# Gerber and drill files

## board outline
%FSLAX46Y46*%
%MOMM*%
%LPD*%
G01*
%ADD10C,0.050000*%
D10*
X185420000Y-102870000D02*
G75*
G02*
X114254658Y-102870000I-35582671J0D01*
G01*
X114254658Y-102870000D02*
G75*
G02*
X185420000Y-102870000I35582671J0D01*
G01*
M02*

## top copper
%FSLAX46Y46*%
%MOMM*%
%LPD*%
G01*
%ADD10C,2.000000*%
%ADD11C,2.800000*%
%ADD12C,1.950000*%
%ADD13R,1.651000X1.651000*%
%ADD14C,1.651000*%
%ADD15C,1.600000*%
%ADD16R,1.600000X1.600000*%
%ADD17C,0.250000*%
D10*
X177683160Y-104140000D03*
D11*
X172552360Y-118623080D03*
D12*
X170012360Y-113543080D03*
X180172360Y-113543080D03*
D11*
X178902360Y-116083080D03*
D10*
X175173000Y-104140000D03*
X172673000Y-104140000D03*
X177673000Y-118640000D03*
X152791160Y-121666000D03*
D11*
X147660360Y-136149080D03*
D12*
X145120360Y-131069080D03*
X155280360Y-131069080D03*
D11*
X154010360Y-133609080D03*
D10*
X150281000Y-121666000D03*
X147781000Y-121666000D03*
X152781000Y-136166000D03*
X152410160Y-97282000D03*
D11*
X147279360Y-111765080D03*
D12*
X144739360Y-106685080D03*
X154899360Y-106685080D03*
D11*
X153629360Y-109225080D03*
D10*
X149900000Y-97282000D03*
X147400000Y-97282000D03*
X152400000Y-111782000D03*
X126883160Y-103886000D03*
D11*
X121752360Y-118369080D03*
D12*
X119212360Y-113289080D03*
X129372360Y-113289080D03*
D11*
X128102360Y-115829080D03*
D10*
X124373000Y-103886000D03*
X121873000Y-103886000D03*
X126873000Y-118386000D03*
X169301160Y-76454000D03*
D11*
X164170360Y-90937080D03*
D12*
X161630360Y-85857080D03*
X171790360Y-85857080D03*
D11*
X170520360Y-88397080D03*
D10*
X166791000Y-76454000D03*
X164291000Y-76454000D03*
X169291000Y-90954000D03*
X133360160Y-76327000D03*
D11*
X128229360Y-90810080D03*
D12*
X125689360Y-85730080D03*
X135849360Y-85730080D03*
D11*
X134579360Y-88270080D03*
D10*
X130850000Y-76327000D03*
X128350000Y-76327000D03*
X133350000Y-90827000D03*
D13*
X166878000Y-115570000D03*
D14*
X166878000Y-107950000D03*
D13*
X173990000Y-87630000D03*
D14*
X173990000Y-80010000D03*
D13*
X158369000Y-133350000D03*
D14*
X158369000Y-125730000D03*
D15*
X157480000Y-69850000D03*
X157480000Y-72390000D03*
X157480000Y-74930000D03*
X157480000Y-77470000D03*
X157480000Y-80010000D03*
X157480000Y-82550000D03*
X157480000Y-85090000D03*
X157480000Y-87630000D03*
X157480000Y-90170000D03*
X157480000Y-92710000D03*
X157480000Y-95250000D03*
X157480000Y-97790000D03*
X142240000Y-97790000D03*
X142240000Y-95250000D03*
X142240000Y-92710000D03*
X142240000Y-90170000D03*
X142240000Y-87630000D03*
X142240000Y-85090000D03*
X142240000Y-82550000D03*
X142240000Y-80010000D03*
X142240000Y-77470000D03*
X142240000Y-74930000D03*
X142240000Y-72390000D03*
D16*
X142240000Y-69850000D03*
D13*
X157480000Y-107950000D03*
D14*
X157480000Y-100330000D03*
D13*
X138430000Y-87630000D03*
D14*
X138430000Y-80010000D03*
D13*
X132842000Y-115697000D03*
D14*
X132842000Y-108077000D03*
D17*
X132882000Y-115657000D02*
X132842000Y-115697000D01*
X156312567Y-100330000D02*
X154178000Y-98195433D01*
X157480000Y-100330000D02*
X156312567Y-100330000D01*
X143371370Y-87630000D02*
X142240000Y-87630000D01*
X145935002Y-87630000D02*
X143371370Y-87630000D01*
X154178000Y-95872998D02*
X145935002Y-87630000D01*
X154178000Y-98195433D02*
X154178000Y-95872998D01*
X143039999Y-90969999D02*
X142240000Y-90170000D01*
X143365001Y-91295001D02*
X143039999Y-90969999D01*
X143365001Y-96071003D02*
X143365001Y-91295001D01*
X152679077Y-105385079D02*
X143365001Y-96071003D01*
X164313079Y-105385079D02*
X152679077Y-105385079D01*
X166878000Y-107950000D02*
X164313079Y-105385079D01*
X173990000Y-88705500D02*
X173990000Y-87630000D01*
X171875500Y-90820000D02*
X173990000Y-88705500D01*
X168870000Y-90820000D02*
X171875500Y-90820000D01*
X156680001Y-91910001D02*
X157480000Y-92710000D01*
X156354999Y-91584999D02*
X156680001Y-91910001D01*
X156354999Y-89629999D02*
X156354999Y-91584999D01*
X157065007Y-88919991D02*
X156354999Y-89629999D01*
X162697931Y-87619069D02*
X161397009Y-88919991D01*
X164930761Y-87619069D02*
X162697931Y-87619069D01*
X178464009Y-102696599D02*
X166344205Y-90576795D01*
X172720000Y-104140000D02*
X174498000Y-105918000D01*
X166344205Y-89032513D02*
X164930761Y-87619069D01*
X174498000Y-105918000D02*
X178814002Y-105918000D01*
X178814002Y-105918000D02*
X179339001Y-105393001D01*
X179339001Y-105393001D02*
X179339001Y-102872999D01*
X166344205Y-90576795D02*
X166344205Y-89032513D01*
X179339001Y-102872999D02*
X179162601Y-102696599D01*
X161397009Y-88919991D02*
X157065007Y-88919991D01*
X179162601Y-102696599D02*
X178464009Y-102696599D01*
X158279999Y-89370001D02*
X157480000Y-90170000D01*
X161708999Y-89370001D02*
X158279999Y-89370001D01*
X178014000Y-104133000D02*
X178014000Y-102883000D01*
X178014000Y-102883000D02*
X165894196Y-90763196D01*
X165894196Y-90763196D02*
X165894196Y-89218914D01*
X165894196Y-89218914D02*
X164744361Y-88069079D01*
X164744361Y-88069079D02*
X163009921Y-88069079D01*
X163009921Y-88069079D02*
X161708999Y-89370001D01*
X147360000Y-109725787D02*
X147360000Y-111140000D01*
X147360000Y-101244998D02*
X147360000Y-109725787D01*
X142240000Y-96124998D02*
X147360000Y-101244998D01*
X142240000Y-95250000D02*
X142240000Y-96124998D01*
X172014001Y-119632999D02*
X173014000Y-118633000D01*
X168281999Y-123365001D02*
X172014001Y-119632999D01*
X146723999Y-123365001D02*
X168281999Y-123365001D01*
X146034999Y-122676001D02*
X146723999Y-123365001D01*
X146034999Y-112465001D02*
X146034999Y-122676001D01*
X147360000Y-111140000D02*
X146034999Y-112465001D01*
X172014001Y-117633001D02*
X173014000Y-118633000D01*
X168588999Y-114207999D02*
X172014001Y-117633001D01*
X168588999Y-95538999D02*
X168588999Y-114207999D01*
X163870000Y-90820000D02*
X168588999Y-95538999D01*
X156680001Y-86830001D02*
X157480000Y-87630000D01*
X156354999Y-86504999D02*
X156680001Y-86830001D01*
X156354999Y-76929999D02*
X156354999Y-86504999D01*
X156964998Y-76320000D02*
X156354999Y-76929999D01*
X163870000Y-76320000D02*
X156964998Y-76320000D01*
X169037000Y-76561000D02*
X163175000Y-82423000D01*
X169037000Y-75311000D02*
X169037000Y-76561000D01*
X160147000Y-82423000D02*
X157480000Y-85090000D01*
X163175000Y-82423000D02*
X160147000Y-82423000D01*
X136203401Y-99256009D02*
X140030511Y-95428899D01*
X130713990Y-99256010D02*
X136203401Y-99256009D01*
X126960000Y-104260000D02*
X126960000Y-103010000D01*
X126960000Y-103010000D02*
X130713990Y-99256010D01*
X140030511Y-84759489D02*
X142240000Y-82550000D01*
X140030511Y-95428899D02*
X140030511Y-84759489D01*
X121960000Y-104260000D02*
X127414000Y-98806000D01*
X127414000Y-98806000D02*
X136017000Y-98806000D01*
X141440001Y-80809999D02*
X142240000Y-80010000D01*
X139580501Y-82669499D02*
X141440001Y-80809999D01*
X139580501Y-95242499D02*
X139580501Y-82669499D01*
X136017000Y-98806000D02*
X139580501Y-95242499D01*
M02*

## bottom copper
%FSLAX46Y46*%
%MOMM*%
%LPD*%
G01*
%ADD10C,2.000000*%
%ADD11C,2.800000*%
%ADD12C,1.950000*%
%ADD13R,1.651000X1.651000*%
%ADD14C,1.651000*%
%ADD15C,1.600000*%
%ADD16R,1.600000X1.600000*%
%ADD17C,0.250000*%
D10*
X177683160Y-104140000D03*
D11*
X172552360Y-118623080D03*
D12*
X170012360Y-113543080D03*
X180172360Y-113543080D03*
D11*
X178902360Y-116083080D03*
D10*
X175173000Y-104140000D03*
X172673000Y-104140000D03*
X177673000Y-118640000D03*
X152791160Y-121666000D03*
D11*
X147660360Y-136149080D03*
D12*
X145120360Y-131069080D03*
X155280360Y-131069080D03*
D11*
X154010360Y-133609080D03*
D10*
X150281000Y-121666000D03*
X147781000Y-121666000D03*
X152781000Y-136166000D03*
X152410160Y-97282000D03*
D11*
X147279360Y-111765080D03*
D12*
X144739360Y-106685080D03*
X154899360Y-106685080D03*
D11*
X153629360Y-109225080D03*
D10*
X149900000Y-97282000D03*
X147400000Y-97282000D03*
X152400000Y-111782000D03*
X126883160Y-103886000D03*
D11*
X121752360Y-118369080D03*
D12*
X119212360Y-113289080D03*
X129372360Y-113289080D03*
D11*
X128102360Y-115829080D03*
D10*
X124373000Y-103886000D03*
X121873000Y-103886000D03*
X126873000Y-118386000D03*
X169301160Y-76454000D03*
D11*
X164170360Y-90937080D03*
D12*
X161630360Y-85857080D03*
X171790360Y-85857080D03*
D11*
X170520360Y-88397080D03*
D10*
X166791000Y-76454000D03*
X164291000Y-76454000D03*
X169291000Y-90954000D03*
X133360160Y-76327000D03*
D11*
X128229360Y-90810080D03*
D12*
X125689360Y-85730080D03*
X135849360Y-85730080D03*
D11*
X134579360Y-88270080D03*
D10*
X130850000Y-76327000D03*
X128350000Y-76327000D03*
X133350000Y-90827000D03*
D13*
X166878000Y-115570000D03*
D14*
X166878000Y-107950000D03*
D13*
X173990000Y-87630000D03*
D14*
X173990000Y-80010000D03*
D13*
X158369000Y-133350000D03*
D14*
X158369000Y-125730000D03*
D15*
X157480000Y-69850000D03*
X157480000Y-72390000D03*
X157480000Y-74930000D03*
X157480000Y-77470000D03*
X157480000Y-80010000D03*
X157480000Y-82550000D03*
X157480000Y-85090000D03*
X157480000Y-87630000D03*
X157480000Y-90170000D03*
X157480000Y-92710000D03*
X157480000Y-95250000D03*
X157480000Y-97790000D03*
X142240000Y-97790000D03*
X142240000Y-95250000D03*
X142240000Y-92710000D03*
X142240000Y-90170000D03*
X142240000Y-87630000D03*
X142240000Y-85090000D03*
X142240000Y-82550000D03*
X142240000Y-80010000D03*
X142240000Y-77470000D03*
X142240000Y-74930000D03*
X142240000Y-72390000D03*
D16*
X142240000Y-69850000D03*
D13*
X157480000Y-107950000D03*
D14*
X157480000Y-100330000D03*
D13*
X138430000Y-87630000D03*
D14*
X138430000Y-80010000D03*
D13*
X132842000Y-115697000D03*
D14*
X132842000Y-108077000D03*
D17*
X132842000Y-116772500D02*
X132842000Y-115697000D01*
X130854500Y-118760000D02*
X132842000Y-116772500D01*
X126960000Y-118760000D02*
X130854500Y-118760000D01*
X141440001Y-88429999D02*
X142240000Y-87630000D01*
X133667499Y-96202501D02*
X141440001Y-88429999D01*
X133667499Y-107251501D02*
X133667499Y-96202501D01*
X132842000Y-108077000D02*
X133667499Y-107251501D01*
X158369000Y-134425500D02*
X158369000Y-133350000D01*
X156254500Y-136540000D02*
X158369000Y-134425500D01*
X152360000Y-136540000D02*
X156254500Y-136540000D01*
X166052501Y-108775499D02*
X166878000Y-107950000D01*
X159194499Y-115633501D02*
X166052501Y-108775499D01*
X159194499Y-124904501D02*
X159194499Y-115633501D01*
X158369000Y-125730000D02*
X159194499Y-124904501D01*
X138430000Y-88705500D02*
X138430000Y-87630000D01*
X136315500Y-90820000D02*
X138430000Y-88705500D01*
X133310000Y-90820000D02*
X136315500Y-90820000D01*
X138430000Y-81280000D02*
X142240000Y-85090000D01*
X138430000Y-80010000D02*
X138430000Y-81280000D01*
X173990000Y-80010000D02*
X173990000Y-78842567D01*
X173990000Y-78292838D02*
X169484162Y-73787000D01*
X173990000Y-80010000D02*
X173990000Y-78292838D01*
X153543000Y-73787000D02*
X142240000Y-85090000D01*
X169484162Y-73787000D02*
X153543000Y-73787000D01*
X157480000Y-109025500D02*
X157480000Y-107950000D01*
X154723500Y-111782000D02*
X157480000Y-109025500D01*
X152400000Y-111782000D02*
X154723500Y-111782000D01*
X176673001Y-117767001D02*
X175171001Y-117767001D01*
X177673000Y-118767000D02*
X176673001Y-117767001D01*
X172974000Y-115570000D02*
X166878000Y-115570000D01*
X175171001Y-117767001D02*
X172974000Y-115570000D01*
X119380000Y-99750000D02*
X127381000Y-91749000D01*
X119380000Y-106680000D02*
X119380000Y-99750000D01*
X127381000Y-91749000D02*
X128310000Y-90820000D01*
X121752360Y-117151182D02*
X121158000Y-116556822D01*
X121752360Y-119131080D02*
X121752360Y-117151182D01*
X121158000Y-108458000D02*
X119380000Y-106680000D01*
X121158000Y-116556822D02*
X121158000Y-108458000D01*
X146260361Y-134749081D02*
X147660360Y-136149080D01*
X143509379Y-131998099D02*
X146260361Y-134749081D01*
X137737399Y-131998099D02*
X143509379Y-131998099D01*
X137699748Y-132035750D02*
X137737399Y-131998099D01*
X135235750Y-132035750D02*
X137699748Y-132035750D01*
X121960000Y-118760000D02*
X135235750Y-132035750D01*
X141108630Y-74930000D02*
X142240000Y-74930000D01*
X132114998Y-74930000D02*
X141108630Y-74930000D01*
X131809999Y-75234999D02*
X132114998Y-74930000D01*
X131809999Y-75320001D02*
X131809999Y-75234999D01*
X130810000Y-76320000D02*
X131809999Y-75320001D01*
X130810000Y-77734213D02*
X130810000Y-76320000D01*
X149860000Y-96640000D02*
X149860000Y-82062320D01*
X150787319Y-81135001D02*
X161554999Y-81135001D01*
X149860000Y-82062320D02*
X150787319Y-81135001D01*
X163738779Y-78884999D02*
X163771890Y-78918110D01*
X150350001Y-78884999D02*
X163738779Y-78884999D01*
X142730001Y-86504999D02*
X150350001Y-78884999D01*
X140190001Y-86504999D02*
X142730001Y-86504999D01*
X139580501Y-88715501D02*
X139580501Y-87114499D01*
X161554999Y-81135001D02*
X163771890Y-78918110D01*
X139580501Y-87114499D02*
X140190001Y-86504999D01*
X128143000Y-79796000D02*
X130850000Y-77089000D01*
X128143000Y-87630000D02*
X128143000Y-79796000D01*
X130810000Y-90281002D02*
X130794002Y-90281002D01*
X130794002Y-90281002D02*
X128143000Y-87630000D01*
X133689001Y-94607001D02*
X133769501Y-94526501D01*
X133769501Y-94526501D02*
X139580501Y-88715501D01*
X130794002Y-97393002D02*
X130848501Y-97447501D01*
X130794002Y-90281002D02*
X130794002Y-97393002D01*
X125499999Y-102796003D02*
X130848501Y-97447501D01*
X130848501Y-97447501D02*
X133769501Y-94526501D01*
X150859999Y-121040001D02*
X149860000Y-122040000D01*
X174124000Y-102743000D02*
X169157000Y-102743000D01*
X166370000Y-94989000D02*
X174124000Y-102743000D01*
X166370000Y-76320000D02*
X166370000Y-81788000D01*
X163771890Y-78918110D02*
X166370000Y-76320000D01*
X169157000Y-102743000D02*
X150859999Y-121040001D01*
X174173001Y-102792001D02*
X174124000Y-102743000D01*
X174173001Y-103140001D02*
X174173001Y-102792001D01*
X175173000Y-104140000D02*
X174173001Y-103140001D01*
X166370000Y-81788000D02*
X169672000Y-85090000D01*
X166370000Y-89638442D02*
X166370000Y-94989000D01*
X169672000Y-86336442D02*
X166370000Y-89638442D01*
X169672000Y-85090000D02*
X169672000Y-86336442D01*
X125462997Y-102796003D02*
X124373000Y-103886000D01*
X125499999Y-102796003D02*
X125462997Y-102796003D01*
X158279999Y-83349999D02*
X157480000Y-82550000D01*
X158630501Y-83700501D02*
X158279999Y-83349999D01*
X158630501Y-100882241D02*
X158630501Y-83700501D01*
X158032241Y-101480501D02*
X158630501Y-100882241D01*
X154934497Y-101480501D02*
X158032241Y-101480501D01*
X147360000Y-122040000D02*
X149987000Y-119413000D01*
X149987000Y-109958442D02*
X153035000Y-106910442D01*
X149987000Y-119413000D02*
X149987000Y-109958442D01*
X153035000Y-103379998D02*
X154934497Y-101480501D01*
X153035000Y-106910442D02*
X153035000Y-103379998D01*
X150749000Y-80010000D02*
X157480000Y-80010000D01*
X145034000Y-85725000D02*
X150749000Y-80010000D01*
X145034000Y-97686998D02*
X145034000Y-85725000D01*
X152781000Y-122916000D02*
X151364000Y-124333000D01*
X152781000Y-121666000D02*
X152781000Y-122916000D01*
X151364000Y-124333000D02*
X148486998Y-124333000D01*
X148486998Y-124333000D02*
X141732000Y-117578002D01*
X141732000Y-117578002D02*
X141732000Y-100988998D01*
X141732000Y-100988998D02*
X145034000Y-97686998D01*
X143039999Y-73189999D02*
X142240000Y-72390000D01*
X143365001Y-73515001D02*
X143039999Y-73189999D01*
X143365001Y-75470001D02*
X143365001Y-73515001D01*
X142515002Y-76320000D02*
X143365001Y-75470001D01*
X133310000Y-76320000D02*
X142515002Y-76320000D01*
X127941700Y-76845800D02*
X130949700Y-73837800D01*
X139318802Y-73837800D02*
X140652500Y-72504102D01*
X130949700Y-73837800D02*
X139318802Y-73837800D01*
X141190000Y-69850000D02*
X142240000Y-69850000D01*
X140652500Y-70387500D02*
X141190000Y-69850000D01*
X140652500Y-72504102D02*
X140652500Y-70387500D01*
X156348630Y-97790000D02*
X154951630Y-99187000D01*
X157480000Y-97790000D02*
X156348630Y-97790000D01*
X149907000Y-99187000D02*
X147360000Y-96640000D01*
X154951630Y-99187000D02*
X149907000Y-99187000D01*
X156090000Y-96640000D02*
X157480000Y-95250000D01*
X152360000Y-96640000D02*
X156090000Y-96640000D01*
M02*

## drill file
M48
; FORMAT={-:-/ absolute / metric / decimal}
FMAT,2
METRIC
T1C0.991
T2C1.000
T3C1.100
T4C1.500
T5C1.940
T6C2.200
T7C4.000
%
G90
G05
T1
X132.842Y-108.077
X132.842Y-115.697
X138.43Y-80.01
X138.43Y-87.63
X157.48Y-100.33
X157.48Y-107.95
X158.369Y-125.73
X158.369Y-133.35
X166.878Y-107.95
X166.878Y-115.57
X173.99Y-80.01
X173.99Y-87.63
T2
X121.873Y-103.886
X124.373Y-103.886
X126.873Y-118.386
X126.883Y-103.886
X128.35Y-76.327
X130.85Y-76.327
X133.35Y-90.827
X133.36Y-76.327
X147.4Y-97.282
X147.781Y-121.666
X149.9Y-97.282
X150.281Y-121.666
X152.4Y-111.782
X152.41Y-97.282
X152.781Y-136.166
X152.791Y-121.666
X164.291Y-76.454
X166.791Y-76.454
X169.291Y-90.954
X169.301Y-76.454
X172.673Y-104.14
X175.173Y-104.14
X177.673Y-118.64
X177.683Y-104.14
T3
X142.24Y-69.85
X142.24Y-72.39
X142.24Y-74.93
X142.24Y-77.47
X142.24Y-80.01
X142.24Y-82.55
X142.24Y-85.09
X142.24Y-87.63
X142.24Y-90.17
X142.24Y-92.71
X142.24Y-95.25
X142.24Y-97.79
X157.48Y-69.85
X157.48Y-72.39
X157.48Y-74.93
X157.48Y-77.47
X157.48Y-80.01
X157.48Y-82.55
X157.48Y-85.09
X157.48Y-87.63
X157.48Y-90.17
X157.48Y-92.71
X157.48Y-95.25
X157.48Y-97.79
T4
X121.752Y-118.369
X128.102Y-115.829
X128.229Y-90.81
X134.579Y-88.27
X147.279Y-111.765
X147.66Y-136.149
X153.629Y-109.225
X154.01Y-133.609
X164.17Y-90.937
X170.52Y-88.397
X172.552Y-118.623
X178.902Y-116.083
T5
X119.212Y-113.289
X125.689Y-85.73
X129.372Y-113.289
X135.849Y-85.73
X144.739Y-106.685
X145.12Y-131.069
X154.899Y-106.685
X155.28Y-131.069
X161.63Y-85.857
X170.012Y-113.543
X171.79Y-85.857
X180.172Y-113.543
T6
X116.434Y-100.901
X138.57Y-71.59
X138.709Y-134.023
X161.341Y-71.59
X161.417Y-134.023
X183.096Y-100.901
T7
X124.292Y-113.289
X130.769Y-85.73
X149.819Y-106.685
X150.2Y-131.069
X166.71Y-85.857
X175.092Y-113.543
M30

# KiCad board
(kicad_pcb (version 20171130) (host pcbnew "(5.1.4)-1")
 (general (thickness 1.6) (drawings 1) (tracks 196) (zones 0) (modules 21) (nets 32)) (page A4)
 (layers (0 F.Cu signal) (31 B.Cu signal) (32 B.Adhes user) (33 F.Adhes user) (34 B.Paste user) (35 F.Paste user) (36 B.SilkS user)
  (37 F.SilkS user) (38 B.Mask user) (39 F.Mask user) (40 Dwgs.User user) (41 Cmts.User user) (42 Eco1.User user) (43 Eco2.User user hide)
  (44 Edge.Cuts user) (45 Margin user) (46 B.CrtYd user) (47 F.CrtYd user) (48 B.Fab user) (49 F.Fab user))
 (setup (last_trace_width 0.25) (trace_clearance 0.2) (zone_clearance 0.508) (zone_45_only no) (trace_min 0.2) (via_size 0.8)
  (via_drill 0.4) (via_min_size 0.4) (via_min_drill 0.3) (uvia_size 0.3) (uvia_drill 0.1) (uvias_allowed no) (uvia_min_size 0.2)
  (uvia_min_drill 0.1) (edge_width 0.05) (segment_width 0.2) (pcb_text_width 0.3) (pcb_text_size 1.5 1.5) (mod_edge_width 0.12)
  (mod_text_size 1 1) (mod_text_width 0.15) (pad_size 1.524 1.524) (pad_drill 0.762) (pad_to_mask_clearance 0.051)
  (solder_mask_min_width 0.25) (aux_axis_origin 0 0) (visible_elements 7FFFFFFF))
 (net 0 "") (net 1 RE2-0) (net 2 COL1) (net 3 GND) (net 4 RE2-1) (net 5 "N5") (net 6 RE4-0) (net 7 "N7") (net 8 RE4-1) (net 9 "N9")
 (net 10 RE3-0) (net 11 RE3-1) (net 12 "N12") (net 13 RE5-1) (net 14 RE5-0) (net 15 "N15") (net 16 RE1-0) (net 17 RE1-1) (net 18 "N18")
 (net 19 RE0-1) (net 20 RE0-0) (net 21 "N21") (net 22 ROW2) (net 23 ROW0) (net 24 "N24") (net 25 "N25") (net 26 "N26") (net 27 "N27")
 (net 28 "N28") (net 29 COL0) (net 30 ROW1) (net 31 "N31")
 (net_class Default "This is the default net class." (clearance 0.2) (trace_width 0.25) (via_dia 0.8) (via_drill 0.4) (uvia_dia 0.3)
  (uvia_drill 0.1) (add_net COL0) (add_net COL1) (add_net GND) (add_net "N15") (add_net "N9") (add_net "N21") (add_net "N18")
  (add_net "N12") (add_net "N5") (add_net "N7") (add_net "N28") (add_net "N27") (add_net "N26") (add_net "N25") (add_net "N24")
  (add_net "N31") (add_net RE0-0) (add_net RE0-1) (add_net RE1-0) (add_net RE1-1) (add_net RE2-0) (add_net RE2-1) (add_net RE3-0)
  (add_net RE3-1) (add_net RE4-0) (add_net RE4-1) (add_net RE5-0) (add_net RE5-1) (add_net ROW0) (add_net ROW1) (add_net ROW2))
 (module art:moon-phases (layer B.Cu) (at 149.7711 102.9208)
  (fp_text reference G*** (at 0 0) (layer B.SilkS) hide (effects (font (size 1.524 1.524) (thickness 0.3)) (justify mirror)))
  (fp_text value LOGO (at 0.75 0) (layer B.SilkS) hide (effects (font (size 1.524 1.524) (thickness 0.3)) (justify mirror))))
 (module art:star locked (layer F.Cu) (at 149.4917 106.6546)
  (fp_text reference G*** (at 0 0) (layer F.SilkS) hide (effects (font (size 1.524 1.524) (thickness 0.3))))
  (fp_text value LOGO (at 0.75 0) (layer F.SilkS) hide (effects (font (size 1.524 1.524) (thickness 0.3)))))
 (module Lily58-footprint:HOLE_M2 (layer F.Cu) (at 161.417 134.0231)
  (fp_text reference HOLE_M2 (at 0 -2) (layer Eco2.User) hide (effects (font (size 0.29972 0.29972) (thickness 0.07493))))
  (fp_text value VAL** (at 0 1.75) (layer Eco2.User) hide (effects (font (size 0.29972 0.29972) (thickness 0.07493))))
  (pad "" np_thru_hole circle (at 0 0) (size 2.2 2.2) (drill 2.2) (layers *.Cu *.Mask F.SilkS) (clearance 0.8)))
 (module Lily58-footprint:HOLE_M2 (layer F.Cu) (at 138.7094 134.0231)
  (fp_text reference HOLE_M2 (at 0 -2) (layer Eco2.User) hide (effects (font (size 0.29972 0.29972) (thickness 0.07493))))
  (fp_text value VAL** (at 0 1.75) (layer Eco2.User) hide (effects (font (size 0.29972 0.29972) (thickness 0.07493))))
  (pad "" np_thru_hole circle (at 0 0) (size 2.2 2.2) (drill 2.2) (layers *.Cu *.Mask F.SilkS) (clearance 0.8)))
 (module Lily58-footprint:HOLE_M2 (layer F.Cu) (at 116.4336 100.9015)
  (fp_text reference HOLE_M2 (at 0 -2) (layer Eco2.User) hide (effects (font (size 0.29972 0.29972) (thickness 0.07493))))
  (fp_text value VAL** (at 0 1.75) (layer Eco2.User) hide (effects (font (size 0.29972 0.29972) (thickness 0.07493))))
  (pad "" np_thru_hole circle (at 0 0) (size 2.2 2.2) (drill 2.2) (layers *.Cu *.Mask F.SilkS) (clearance 0.8)))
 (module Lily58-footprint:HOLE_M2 (layer F.Cu) (at 183.0959 100.9015)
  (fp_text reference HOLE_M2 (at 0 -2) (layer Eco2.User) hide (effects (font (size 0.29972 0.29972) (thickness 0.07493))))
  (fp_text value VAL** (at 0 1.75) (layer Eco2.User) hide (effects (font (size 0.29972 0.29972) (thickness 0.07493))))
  (pad "" np_thru_hole circle (at 0 0) (size 2.2 2.2) (drill 2.2) (layers *.Cu *.Mask F.SilkS) (clearance 0.8)))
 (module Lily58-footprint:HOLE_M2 (layer F.Cu) (at 138.5697 71.5899)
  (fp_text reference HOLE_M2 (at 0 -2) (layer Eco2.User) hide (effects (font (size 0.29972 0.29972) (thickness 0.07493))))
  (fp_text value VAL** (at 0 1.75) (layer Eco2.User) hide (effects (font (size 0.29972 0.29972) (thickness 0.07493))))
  (pad "" np_thru_hole circle (at 0 0) (size 2.2 2.2) (drill 2.2) (layers *.Cu *.Mask F.SilkS) (clearance 0.8)))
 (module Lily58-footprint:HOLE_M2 (layer F.Cu) (at 161.3408 71.5899)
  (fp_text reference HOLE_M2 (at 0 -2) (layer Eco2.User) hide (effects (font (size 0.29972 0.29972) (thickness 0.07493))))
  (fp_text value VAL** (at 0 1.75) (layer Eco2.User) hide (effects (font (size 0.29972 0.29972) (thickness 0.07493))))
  (pad "" np_thru_hole circle (at 0 0) (size 2.2 2.2) (drill 2.2) (layers *.Cu *.Mask F.SilkS) (clearance 0.8)))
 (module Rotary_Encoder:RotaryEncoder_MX (layer F.Cu) (at 177.673 104.14 270)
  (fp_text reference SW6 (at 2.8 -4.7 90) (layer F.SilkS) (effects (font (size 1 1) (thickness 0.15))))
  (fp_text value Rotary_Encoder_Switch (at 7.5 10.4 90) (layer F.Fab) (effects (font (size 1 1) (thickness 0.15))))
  (pad A thru_hole circle (at 0 -0.01016 270) (size 2 2) (drill 1) (layers *.Cu *.Mask) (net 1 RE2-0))
  (pad S1 thru_hole circle (at 14.48308 5.12064 180) (size 2.8 2.8) (drill 1.5) (layers *.Cu *.Mask) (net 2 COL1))
  (pad "" np_thru_hole circle (at 9.40308 7.66064 180) (size 1.95 1.95) (drill 1.94) (layers *.Cu *.Mask) (clearance 0.1524))
  (pad "" np_thru_hole circle (at 9.40308 -2.49936 180) (size 1.95 1.95) (drill 1.94) (layers *.Cu *.Mask) (clearance 0.1524))
  (pad "" np_thru_hole circle (at 9.40308 2.58064 180) (size 4 4) (drill 4) (layers *.Cu *.Mask) (clearance 0.1524))
  (pad S2_2 thru_hole circle (at 11.94308 -1.22936 180) (size 2.8 2.8) (drill 1.5) (layers *.Cu *.Mask))
  (pad C thru_hole circle (at 0 2.5 270) (size 2 2) (drill 1) (layers *.Cu *.Mask) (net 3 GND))
  (pad B thru_hole circle (at 0 5 270) (size 2 2) (drill 1) (layers *.Cu *.Mask) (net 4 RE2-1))
  (pad S2 thru_hole circle (at 14.5 0 270) (size 2 2) (drill 1) (layers *.Cu *.Mask) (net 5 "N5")))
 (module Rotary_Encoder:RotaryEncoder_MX (layer F.Cu) (at 152.781 121.666 270)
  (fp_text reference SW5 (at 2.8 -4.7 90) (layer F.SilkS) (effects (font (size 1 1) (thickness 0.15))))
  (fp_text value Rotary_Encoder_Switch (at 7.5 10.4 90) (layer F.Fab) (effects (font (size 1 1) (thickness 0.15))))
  (pad A thru_hole circle (at 0 -0.01016 270) (size 2 2) (drill 1) (layers *.Cu *.Mask) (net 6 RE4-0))
  (pad S1 thru_hole circle (at 14.48308 5.12064 180) (size 2.8 2.8) (drill 1.5) (layers *.Cu *.Mask) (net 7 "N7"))
  (pad "" np_thru_hole circle (at 9.40308 7.66064 180) (size 1.95 1.95) (drill 1.94) (layers *.Cu *.Mask) (clearance 0.1524))
  (pad "" np_thru_hole circle (at 9.40308 -2.49936 180) (size 1.95 1.95) (drill 1.94) (layers *.Cu *.Mask) (clearance 0.1524))
  (pad "" np_thru_hole circle (at 9.40308 2.58064 180) (size 4 4) (drill 4) (layers *.Cu *.Mask) (clearance 0.1524))
  (pad S2_2 thru_hole circle (at 11.94308 -1.22936 180) (size 2.8 2.8) (drill 1.5) (layers *.Cu *.Mask))
  (pad C thru_hole circle (at 0 2.5 270) (size 2 2) (drill 1) (layers *.Cu *.Mask) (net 3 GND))
  (pad B thru_hole circle (at 0 5 270) (size 2 2) (drill 1) (layers *.Cu *.Mask) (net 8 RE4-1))
  (pad S2 thru_hole circle (at 14.5 0 270) (size 2 2) (drill 1) (layers *.Cu *.Mask) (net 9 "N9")))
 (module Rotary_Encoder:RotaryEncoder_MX (layer F.Cu) (at 152.4 97.282 270)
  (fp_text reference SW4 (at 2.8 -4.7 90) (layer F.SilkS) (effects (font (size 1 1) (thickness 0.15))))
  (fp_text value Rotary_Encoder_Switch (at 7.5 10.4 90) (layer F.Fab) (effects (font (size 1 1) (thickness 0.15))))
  (pad A thru_hole circle (at 0 -0.01016 270) (size 2 2) (drill 1) (layers *.Cu *.Mask) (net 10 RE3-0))
  (pad S1 thru_hole circle (at 14.48308 5.12064 180) (size 2.8 2.8) (drill 1.5) (layers *.Cu *.Mask) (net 2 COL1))
  (pad "" np_thru_hole circle (at 9.40308 7.66064 180) (size 1.95 1.95) (drill 1.94) (layers *.Cu *.Mask) (clearance 0.1524))
  (pad "" np_thru_hole circle (at 9.40308 -2.49936 180) (size 1.95 1.95) (drill 1.94) (layers *.Cu *.Mask) (clearance 0.1524))
  (pad "" np_thru_hole circle (at 9.40308 2.58064 180) (size 4 4) (drill 4) (layers *.Cu *.Mask) (clearance 0.1524))
  (pad S2_2 thru_hole circle (at 11.94308 -1.22936 180) (size 2.8 2.8) (drill 1.5) (layers *.Cu *.Mask))
  (pad C thru_hole circle (at 0 2.5 270) (size 2 2) (drill 1) (layers *.Cu *.Mask) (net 3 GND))
  (pad B thru_hole circle (at 0 5 270) (size 2 2) (drill 1) (layers *.Cu *.Mask) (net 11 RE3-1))
  (pad S2 thru_hole circle (at 14.5 0 270) (size 2 2) (drill 1) (layers *.Cu *.Mask) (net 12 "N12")))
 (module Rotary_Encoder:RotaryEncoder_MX (layer F.Cu) (at 126.873 103.886 270)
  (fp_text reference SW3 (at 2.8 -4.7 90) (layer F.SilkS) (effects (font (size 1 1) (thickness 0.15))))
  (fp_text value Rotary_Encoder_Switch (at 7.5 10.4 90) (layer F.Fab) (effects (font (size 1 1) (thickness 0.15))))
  (pad A thru_hole circle (at 0 -0.01016 270) (size 2 2) (drill 1) (layers *.Cu *.Mask) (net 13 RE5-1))
  (pad S1 thru_hole circle (at 14.48308 5.12064 180) (size 2.8 2.8) (drill 1.5) (layers *.Cu *.Mask) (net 7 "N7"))
  (pad "" np_thru_hole circle (at 9.40308 7.66064 180) (size 1.95 1.95) (drill 1.94) (layers *.Cu *.Mask) (clearance 0.1524))
  (pad "" np_thru_hole circle (at 9.40308 -2.49936 180) (size 1.95 1.95) (drill 1.94) (layers *.Cu *.Mask) (clearance 0.1524))
  (pad "" np_thru_hole circle (at 9.40308 2.58064 180) (size 4 4) (drill 4) (layers *.Cu *.Mask) (clearance 0.1524))
  (pad S2_2 thru_hole circle (at 11.94308 -1.22936 180) (size 2.8 2.8) (drill 1.5) (layers *.Cu *.Mask))
  (pad C thru_hole circle (at 0 2.5 270) (size 2 2) (drill 1) (layers *.Cu *.Mask) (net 3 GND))
  (pad B thru_hole circle (at 0 5 270) (size 2 2) (drill 1) (layers *.Cu *.Mask) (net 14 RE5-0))
  (pad S2 thru_hole circle (at 14.5 0 270) (size 2 2) (drill 1) (layers *.Cu *.Mask) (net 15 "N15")))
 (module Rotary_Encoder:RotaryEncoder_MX (layer F.Cu) (at 169.291 76.454 270)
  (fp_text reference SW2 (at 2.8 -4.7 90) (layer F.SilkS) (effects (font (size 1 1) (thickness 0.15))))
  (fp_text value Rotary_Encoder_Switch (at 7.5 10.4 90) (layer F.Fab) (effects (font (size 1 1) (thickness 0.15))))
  (pad A thru_hole circle (at 0 -0.01016 270) (size 2 2) (drill 1) (layers *.Cu *.Mask) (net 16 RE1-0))
  (pad S1 thru_hole circle (at 14.48308 5.12064 180) (size 2.8 2.8) (drill 1.5) (layers *.Cu *.Mask) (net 2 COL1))
  (pad "" np_thru_hole circle (at 9.40308 7.66064 180) (size 1.95 1.95) (drill 1.94) (layers *.Cu *.Mask) (clearance 0.1524))
  (pad "" np_thru_hole circle (at 9.40308 -2.49936 180) (size 1.95 1.95) (drill 1.94) (layers *.Cu *.Mask) (clearance 0.1524))
  (pad "" np_thru_hole circle (at 9.40308 2.58064 180) (size 4 4) (drill 4) (layers *.Cu *.Mask) (clearance 0.1524))
  (pad S2_2 thru_hole circle (at 11.94308 -1.22936 180) (size 2.8 2.8) (drill 1.5) (layers *.Cu *.Mask))
  (pad C thru_hole circle (at 0 2.5 270) (size 2 2) (drill 1) (layers *.Cu *.Mask) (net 3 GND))
  (pad B thru_hole circle (at 0 5 270) (size 2 2) (drill 1) (layers *.Cu *.Mask) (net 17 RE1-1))
  (pad S2 thru_hole circle (at 14.5 0 270) (size 2 2) (drill 1) (layers *.Cu *.Mask) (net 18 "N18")))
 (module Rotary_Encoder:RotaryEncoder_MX (layer F.Cu) (at 133.35 76.327 270)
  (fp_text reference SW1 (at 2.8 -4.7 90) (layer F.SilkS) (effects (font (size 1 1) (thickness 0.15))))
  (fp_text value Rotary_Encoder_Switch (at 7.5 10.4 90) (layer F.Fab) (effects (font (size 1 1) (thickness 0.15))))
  (pad A thru_hole circle (at 0 -0.01016 270) (size 2 2) (drill 1) (layers *.Cu *.Mask) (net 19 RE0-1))
  (pad S1 thru_hole circle (at 14.48308 5.12064 180) (size 2.8 2.8) (drill 1.5) (layers *.Cu *.Mask) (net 7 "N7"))
  (pad "" np_thru_hole circle (at 9.40308 7.66064 180) (size 1.95 1.95) (drill 1.94) (layers *.Cu *.Mask) (clearance 0.1524))
  (pad "" np_thru_hole circle (at 9.40308 -2.49936 180) (size 1.95 1.95) (drill 1.94) (layers *.Cu *.Mask) (clearance 0.1524))
  (pad "" np_thru_hole circle (at 9.40308 2.58064 180) (size 4 4) (drill 4) (layers *.Cu *.Mask) (clearance 0.1524))
  (pad S2_2 thru_hole circle (at 11.94308 -1.22936 180) (size 2.8 2.8) (drill 1.5) (layers *.Cu *.Mask))
  (pad C thru_hole circle (at 0 2.5 270) (size 2 2) (drill 1) (layers *.Cu *.Mask) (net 3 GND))
  (pad B thru_hole circle (at 0 5 270) (size 2 2) (drill 1) (layers *.Cu *.Mask) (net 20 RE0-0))
  (pad S2 thru_hole circle (at 14.5 0 270) (size 2 2) (drill 1) (layers *.Cu *.Mask) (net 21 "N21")))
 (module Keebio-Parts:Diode (layer F.Cu) (at 166.878 111.76 270)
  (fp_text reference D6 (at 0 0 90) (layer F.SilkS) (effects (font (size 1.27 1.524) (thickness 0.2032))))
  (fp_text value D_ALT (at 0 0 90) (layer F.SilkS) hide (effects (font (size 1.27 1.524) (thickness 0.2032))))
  (pad 2 thru_hole rect (at 3.81 0 270) (size 1.651 1.651) (drill 0.9906) (layers *.Cu *.SilkS *.Mask) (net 5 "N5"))
  (pad 1 thru_hole circle (at -3.81 0 270) (size 1.651 1.651) (drill 0.9906) (layers *.Cu *.SilkS *.Mask) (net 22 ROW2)))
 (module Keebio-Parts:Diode (layer F.Cu) (at 173.99 83.82 270)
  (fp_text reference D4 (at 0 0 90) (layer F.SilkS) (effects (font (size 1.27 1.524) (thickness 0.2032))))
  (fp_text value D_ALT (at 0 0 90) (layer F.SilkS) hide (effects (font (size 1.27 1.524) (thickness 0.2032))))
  (pad 2 thru_hole rect (at 3.81 0 270) (size 1.651 1.651) (drill 0.9906) (layers *.Cu *.SilkS *.Mask) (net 18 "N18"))
  (pad 1 thru_hole circle (at -3.81 0 270) (size 1.651 1.651) (drill 0.9906) (layers *.Cu *.SilkS *.Mask) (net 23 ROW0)))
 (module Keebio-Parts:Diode (layer F.Cu) (at 158.369 129.54 270)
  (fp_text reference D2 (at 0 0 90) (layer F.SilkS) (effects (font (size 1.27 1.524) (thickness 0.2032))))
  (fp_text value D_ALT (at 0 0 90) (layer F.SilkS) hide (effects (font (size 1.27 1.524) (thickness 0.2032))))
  (pad 2 thru_hole rect (at 3.81 0 270) (size 1.651 1.651) (drill 0.9906) (layers *.Cu *.SilkS *.Mask) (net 9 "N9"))
  (pad 1 thru_hole circle (at -3.81 0 270) (size 1.651 1.651) (drill 0.9906) (layers *.Cu *.SilkS *.Mask) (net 22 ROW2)))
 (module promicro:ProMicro (layer F.Cu) (at 149.86 83.82 270)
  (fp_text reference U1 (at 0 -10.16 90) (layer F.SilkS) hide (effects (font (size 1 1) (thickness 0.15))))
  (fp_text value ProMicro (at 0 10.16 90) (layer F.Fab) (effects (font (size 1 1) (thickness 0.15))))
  (pad 24 thru_hole circle (at -13.97 -7.62 270) (size 1.6 1.6) (drill 1.1) (layers *.Cu *.Mask F.SilkS) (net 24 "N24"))
  (pad 23 thru_hole circle (at -11.43 -7.62 270) (size 1.6 1.6) (drill 1.1) (layers *.Cu *.Mask F.SilkS) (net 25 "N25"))
  (pad 22 thru_hole circle (at -8.89 -7.62 270) (size 1.6 1.6) (drill 1.1) (layers *.Cu *.Mask F.SilkS) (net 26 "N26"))
  (pad 21 thru_hole circle (at -6.35 -7.62 270) (size 1.6 1.6) (drill 1.1) (layers *.Cu *.Mask F.SilkS) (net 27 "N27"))
  (pad 20 thru_hole circle (at -3.81 -7.62 270) (size 1.6 1.6) (drill 1.1) (layers *.Cu *.Mask F.SilkS) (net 6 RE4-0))
  (pad 19 thru_hole circle (at -1.27 -7.62 270) (size 1.6 1.6) (drill 1.1) (layers *.Cu *.Mask F.SilkS) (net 8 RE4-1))
  (pad 18 thru_hole circle (at 1.27 -7.62 270) (size 1.6 1.6) (drill 1.1) (layers *.Cu *.Mask F.SilkS) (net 16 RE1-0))
  (pad 17 thru_hole circle (at 3.81 -7.62 270) (size 1.6 1.6) (drill 1.1) (layers *.Cu *.Mask F.SilkS) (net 17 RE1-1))
  (pad 16 thru_hole circle (at 6.35 -7.62 270) (size 1.6 1.6) (drill 1.1) (layers *.Cu *.Mask F.SilkS) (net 1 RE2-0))
  (pad 15 thru_hole circle (at 8.89 -7.62 270) (size 1.6 1.6) (drill 1.1) (layers *.Cu *.Mask F.SilkS) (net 4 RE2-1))
  (pad 14 thru_hole circle (at 11.43 -7.62 270) (size 1.6 1.6) (drill 1.1) (layers *.Cu *.Mask F.SilkS) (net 10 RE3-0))
  (pad 13 thru_hole circle (at 13.97 -7.62 270) (size 1.6 1.6) (drill 1.1) (layers *.Cu *.Mask F.SilkS) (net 11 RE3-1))
  (pad 12 thru_hole circle (at 13.97 7.62 270) (size 1.6 1.6) (drill 1.1) (layers *.Cu *.Mask F.SilkS) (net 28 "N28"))
  (pad 11 thru_hole circle (at 11.43 7.62 270) (size 1.6 1.6) (drill 1.1) (layers *.Cu *.Mask F.SilkS) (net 2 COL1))
  (pad 10 thru_hole circle (at 8.89 7.62 270) (size 1.6 1.6) (drill 1.1) (layers *.Cu *.Mask F.SilkS) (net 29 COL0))
  (pad 9 thru_hole circle (at 6.35 7.62 270) (size 1.6 1.6) (drill 1.1) (layers *.Cu *.Mask F.SilkS) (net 22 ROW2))
  (pad 8 thru_hole circle (at 3.81 7.62 270) (size 1.6 1.6) (drill 1.1) (layers *.Cu *.Mask F.SilkS) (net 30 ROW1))
  (pad 7 thru_hole circle (at 1.27 7.62 270) (size 1.6 1.6) (drill 1.1) (layers *.Cu *.Mask F.SilkS) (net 23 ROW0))
  (pad 6 thru_hole circle (at -1.27 7.62 270) (size 1.6 1.6) (drill 1.1) (layers *.Cu *.Mask F.SilkS) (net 13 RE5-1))
  (pad 5 thru_hole circle (at -3.81 7.62 270) (size 1.6 1.6) (drill 1.1) (layers *.Cu *.Mask F.SilkS) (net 14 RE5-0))
  (pad 4 thru_hole circle (at -6.35 7.62 270) (size 1.6 1.6) (drill 1.1) (layers *.Cu *.Mask F.SilkS) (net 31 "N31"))
  (pad 3 thru_hole circle (at -8.89 7.62 270) (size 1.6 1.6) (drill 1.1) (layers *.Cu *.Mask F.SilkS) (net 3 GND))
  (pad 2 thru_hole circle (at -11.43 7.62 270) (size 1.6 1.6) (drill 1.1) (layers *.Cu *.Mask F.SilkS) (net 19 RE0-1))
  (pad 1 thru_hole rect (at -13.97 7.62 270) (size 1.6 1.6) (drill 1.1) (layers *.Cu *.Mask F.SilkS) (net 20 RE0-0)))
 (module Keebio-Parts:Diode (layer F.Cu) (at 157.48 104.14 270)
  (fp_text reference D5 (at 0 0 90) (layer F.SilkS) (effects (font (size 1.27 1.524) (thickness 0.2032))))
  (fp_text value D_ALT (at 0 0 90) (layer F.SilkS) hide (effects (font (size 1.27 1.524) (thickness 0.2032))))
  (pad 2 thru_hole rect (at 3.81 0 270) (size 1.651 1.651) (drill 0.9906) (layers *.Cu *.SilkS *.Mask) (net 12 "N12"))
  (pad 1 thru_hole circle (at -3.81 0 270) (size 1.651 1.651) (drill 0.9906) (layers *.Cu *.SilkS *.Mask) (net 30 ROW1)))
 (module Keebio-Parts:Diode (layer F.Cu) (at 138.43 83.82 270)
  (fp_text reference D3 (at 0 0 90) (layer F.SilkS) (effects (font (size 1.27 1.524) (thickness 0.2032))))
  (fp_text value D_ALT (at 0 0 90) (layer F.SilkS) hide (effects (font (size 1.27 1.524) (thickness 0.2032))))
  (pad 2 thru_hole rect (at 3.81 0 270) (size 1.651 1.651) (drill 0.9906) (layers *.Cu *.SilkS *.Mask) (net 21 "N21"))
  (pad 1 thru_hole circle (at -3.81 0 270) (size 1.651 1.651) (drill 0.9906) (layers *.Cu *.SilkS *.Mask) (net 23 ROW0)))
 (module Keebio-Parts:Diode (layer F.Cu) (at 132.842 111.887 270)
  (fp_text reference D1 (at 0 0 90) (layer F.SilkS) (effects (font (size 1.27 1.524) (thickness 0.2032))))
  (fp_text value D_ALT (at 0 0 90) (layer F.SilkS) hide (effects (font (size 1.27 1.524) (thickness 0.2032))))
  (pad 2 thru_hole rect (at 3.81 0 270) (size 1.651 1.651) (drill 0.9906) (layers *.Cu *.SilkS *.Mask) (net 15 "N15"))
  (pad 1 thru_hole circle (at -3.81 0 270) (size 1.651 1.651) (drill 0.9906) (layers *.Cu *.SilkS *.Mask) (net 30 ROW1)))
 (gr_circle (center 149.837329 102.87) (end 185.397329 104.14) (layer Edge.Cuts) (width 0.05))
 (segment (start 132.882 115.657) (end 132.842 115.697) (width 0.25) (layer F.Cu) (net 15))
 (segment (start 132.842 116.7725) (end 132.842 115.697) (width 0.25) (layer B.Cu) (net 15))
 (segment (start 130.8545 118.76) (end 132.842 116.7725) (width 0.25) (layer B.Cu) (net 15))
 (segment (start 126.96 118.76) (end 130.8545 118.76) (width 0.25) (layer B.Cu) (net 15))
 (segment (start 141.440001 88.429999) (end 142.24 87.63) (width 0.25) (layer B.Cu) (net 30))
 (segment (start 133.667499 96.202501) (end 141.440001 88.429999) (width 0.25) (layer B.Cu) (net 30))
 (segment (start 133.667499 107.251501) (end 133.667499 96.202501) (width 0.25) (layer B.Cu) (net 30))
 (segment (start 132.842 108.077) (end 133.667499 107.251501) (width 0.25) (layer B.Cu) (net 30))
 (segment (start 156.312567 100.33) (end 154.178 98.195433) (width 0.25) (layer F.Cu) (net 30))
 (segment (start 157.48 100.33) (end 156.312567 100.33) (width 0.25) (layer F.Cu) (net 30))
 (segment (start 143.37137 87.63) (end 142.24 87.63) (width 0.25) (layer F.Cu) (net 30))
 (segment (start 145.935002 87.63) (end 143.37137 87.63) (width 0.25) (layer F.Cu) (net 30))
 (segment (start 154.178 95.872998) (end 145.935002 87.63) (width 0.25) (layer F.Cu) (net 30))
 (segment (start 154.178 98.195433) (end 154.178 95.872998) (width 0.25) (layer F.Cu) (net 30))
 (segment (start 158.369 134.4255) (end 158.369 133.35) (width 0.25) (layer B.Cu) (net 9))
 (segment (start 156.2545 136.54) (end 158.369 134.4255) (width 0.25) (layer B.Cu) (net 9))
 (segment (start 152.36 136.54) (end 156.2545 136.54) (width 0.25) (layer B.Cu) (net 9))
 (segment (start 166.052501 108.775499) (end 166.878 107.95) (width 0.25) (layer B.Cu) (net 22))
 (segment (start 159.194499 115.633501) (end 166.052501 108.775499) (width 0.25) (layer B.Cu) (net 22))
 (segment (start 159.194499 124.904501) (end 159.194499 115.633501) (width 0.25) (layer B.Cu) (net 22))
 (segment (start 158.369 125.73) (end 159.194499 124.904501) (width 0.25) (layer B.Cu) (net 22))
 (segment (start 143.039999 90.969999) (end 142.24 90.17) (width 0.25) (layer F.Cu) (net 22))
 (segment (start 143.365001 91.295001) (end 143.039999 90.969999) (width 0.25) (layer F.Cu) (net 22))
 (segment (start 143.365001 96.071003) (end 143.365001 91.295001) (width 0.25) (layer F.Cu) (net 22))
 (segment (start 152.679077 105.385079) (end 143.365001 96.071003) (width 0.25) (layer F.Cu) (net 22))
 (segment (start 164.313079 105.385079) (end 152.679077 105.385079) (width 0.25) (layer F.Cu) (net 22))
 (segment (start 166.878 107.95) (end 164.313079 105.385079) (width 0.25) (layer F.Cu) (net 22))
 (segment (start 138.43 88.7055) (end 138.43 87.63) (width 0.25) (layer B.Cu) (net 21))
 (segment (start 136.3155 90.82) (end 138.43 88.7055) (width 0.25) (layer B.Cu) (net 21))
 (segment (start 133.31 90.82) (end 136.3155 90.82) (width 0.25) (layer B.Cu) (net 21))
 (segment (start 138.43 81.28) (end 142.24 85.09) (width 0.25) (layer B.Cu) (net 23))
 (segment (start 138.43 80.01) (end 138.43 81.28) (width 0.25) (layer B.Cu) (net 23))
 (segment (start 173.99 80.01) (end 173.99 78.842567) (width 0.25) (layer B.Cu) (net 23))
 (segment (start 173.99 78.292838) (end 169.484162 73.787) (width 0.25) (layer B.Cu) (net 23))
 (segment (start 173.99 80.01) (end 173.99 78.292838) (width 0.25) (layer B.Cu) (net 23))
 (segment (start 153.543 73.787) (end 142.24 85.09) (width 0.25) (layer B.Cu) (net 23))
 (segment (start 169.484162 73.787) (end 153.543 73.787) (width 0.25) (layer B.Cu) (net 23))
 (segment (start 173.99 88.7055) (end 173.99 87.63) (width 0.25) (layer F.Cu) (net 18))
 (segment (start 171.8755 90.82) (end 173.99 88.7055) (width 0.25) (layer F.Cu) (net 18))
 (segment (start 168.87 90.82) (end 171.8755 90.82) (width 0.25) (layer F.Cu) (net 18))
 (segment (start 157.48 109.0255) (end 157.48 107.95) (width 0.25) (layer B.Cu) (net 12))
 (segment (start 154.7235 111.782) (end 157.48 109.0255) (width 0.25) (layer B.Cu) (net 12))
 (segment (start 152.4 111.782) (end 154.7235 111.782) (width 0.25) (layer B.Cu) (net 12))
 (segment (start 176.673001 117.767001) (end 175.171001 117.767001) (width 0.25) (layer B.Cu) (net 5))
 (segment (start 177.673 118.767) (end 176.673001 117.767001) (width 0.25) (layer B.Cu) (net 5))
 (segment (start 172.974 115.57) (end 166.878 115.57) (width 0.25) (layer B.Cu) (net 5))
 (segment (start 175.171001 117.767001) (end 172.974 115.57) (width 0.25) (layer B.Cu) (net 5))
 (segment (start 119.38 99.75) (end 127.381 91.749) (width 0.25) (layer B.Cu) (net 7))
 (segment (start 119.38 106.68) (end 119.38 99.75) (width 0.25) (layer B.Cu) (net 7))
 (segment (start 127.381 91.749) (end 128.31 90.82) (width 0.25) (layer B.Cu) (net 7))
 (segment (start 121.75236 117.151182) (end 121.158 116.556822) (width 0.25) (layer B.Cu) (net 7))
 (segment (start 121.75236 119.13108) (end 121.75236 117.151182) (width 0.25) (layer B.Cu) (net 7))
 (segment (start 121.158 108.458) (end 119.38 106.68) (width 0.25) (layer B.Cu) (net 7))
 (segment (start 121.158 116.556822) (end 121.158 108.458) (width 0.25) (layer B.Cu) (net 7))
 (segment (start 146.260361 134.749081) (end 147.66036 136.14908) (width 0.25) (layer B.Cu) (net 7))
 (segment (start 143.509379 131.998099) (end 146.260361 134.749081) (width 0.25) (layer B.Cu) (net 7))
 (segment (start 137.737399 131.998099) (end 143.509379 131.998099) (width 0.25) (layer B.Cu) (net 7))
 (segment (start 137.699748 132.03575) (end 137.737399 131.998099) (width 0.25) (layer B.Cu) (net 7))
 (segment (start 135.23575 132.03575) (end 137.699748 132.03575) (width 0.25) (layer B.Cu) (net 7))
 (segment (start 121.96 118.76) (end 135.23575 132.03575) (width 0.25) (layer B.Cu) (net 7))
 (segment (start 156.680001 91.910001) (end 157.48 92.71) (width 0.25) (layer F.Cu) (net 4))
 (segment (start 156.354999 91.584999) (end 156.680001 91.910001) (width 0.25) (layer F.Cu) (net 4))
 (segment (start 156.354999 89.629999) (end 156.354999 91.584999) (width 0.25) (layer F.Cu) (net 4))
 (segment (start 157.065007 88.919991) (end 156.354999 89.629999) (width 0.25) (layer F.Cu) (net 4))
 (segment (start 162.697931 87.619069) (end 161.397009 88.919991) (width 0.25) (layer F.Cu) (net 4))
 (segment (start 164.930761 87.619069) (end 162.697931 87.619069) (width 0.25) (layer F.Cu) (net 4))
 (segment (start 178.464009 102.696599) (end 166.344205 90.576795) (width 0.25) (layer F.Cu) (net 4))
 (segment (start 172.72 104.14) (end 174.498 105.918) (width 0.25) (layer F.Cu) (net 4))
 (segment (start 166.344205 89.032513) (end 164.930761 87.619069) (width 0.25) (layer F.Cu) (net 4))
 (segment (start 174.498 105.918) (end 178.814002 105.918) (width 0.25) (layer F.Cu) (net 4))
 (segment (start 178.814002 105.918) (end 179.339001 105.393001) (width 0.25) (layer F.Cu) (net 4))
 (segment (start 179.339001 105.393001) (end 179.339001 102.872999) (width 0.25) (layer F.Cu) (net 4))
 (segment (start 166.344205 90.576795) (end 166.344205 89.032513) (width 0.25) (layer F.Cu) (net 4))
 (segment (start 179.339001 102.872999) (end 179.162601 102.696599) (width 0.25) (layer F.Cu) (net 4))
 (segment (start 161.397009 88.919991) (end 157.065007 88.919991) (width 0.25) (layer F.Cu) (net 4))
 (segment (start 179.162601 102.696599) (end 178.464009 102.696599) (width 0.25) (layer F.Cu) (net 4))
 (segment (start 141.10863 74.93) (end 142.24 74.93) (width 0.25) (layer B.Cu) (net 3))
 (segment (start 132.114998 74.93) (end 141.10863 74.93) (width 0.25) (layer B.Cu) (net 3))
 (segment (start 131.809999 75.234999) (end 132.114998 74.93) (width 0.25) (layer B.Cu) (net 3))
 (segment (start 131.809999 75.320001) (end 131.809999 75.234999) (width 0.25) (layer B.Cu) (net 3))
 (segment (start 130.81 76.32) (end 131.809999 75.320001) (width 0.25) (layer B.Cu) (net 3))
 (segment (start 130.81 77.734213) (end 130.81 76.32) (width 0.25) (layer B.Cu) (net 3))
 (segment (start 149.86 96.64) (end 149.86 82.06232) (width 0.25) (layer B.Cu) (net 3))
 (segment (start 150.787319 81.135001) (end 161.554999 81.135001) (width 0.25) (layer B.Cu) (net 3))
 (segment (start 149.86 82.06232) (end 150.787319 81.135001) (width 0.25) (layer B.Cu) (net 3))
 (segment (start 163.738779 78.884999) (end 163.77189 78.91811) (width 0.25) (layer B.Cu) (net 3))
 (segment (start 150.350001 78.884999) (end 163.738779 78.884999) (width 0.25) (layer B.Cu) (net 3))
 (segment (start 142.730001 86.504999) (end 150.350001 78.884999) (width 0.25) (layer B.Cu) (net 3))
 (segment (start 140.190001 86.504999) (end 142.730001 86.504999) (width 0.25) (layer B.Cu) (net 3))
 (segment (start 139.580501 88.715501) (end 139.580501 87.114499) (width 0.25) (layer B.Cu) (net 3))
 (segment (start 161.554999 81.135001) (end 163.77189 78.91811) (width 0.25) (layer B.Cu) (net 3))
 (segment (start 139.580501 87.114499) (end 140.190001 86.504999) (width 0.25) (layer B.Cu) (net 3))
 (segment (start 128.143 79.796) (end 130.85 77.089) (width 0.25) (layer B.Cu) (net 3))
 (segment (start 128.143 87.63) (end 128.143 79.796) (width 0.25) (layer B.Cu) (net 3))
 (segment (start 130.81 90.281002) (end 130.794002 90.281002) (width 0.25) (layer B.Cu) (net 3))
 (segment (start 130.794002 90.281002) (end 128.143 87.63) (width 0.25) (layer B.Cu) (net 3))
 (segment (start 133.689001 94.607001) (end 133.769501 94.526501) (width 0.25) (layer B.Cu) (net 3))
 (segment (start 133.769501 94.526501) (end 139.580501 88.715501) (width 0.25) (layer B.Cu) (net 3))
 (segment (start 130.794002 97.393002) (end 130.848501 97.447501) (width 0.25) (layer B.Cu) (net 3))
 (segment (start 130.794002 90.281002) (end 130.794002 97.393002) (width 0.25) (layer B.Cu) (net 3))
 (segment (start 125.499999 102.796003) (end 130.848501 97.447501) (width 0.25) (layer B.Cu) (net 3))
 (segment (start 130.848501 97.447501) (end 133.769501 94.526501) (width 0.25) (layer B.Cu) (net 3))
 (segment (start 150.859999 121.040001) (end 149.86 122.04) (width 0.25) (layer B.Cu) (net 3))
 (segment (start 174.124 102.743) (end 169.157 102.743) (width 0.25) (layer B.Cu) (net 3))
 (segment (start 166.37 94.989) (end 174.124 102.743) (width 0.25) (layer B.Cu) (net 3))
 (segment (start 166.37 76.32) (end 166.37 81.788) (width 0.25) (layer B.Cu) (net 3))
 (segment (start 163.77189 78.91811) (end 166.37 76.32) (width 0.25) (layer B.Cu) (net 3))
 (segment (start 169.157 102.743) (end 150.859999 121.040001) (width 0.25) (layer B.Cu) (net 3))
 (segment (start 174.173001 102.792001) (end 174.124 102.743) (width 0.25) (layer B.Cu) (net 3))
 (segment (start 174.173001 103.140001) (end 174.173001 102.792001) (width 0.25) (layer B.Cu) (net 3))
 (segment (start 175.173 104.14) (end 174.173001 103.140001) (width 0.25) (layer B.Cu) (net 3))
 (segment (start 166.37 81.788) (end 169.672 85.09) (width 0.25) (layer B.Cu) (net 3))
 (segment (start 166.37 89.638442) (end 166.37 94.989) (width 0.25) (layer B.Cu) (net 3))
 (segment (start 169.672 86.336442) (end 166.37 89.638442) (width 0.25) (layer B.Cu) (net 3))
 (segment (start 169.672 85.09) (end 169.672 86.336442) (width 0.25) (layer B.Cu) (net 3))
 (segment (start 125.462997 102.796003) (end 124.373 103.886) (width 0.25) (layer B.Cu) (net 3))
 (segment (start 125.499999 102.796003) (end 125.462997 102.796003) (width 0.25) (layer B.Cu) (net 3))
 (segment (start 158.279999 89.370001) (end 157.48 90.17) (width 0.25) (layer F.Cu) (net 1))
 (segment (start 161.708999 89.370001) (end 158.279999 89.370001) (width 0.25) (layer F.Cu) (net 1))
 (segment (start 178.014 104.133) (end 178.014 102.883) (width 0.25) (layer F.Cu) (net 1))
 (segment (start 178.014 102.883) (end 165.894196 90.763196) (width 0.25) (layer F.Cu) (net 1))
 (segment (start 165.894196 90.763196) (end 165.894196 89.218914) (width 0.25) (layer F.Cu) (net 1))
 (segment (start 165.894196 89.218914) (end 164.744361 88.069079) (width 0.25) (layer F.Cu) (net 1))
 (segment (start 164.744361 88.069079) (end 163.009921 88.069079) (width 0.25) (layer F.Cu) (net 1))
 (segment (start 163.009921 88.069079) (end 161.708999 89.370001) (width 0.25) (layer F.Cu) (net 1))
 (segment (start 158.279999 83.349999) (end 157.48 82.55) (width 0.25) (layer B.Cu) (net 8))
 (segment (start 158.630501 83.700501) (end 158.279999 83.349999) (width 0.25) (layer B.Cu) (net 8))
 (segment (start 158.630501 100.882241) (end 158.630501 83.700501) (width 0.25) (layer B.Cu) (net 8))
 (segment (start 158.032241 101.480501) (end 158.630501 100.882241) (width 0.25) (layer B.Cu) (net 8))
 (segment (start 154.934497 101.480501) (end 158.032241 101.480501) (width 0.25) (layer B.Cu) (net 8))
 (segment (start 147.36 122.04) (end 149.987 119.413) (width 0.25) (layer B.Cu) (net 8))
 (segment (start 149.987 109.958442) (end 153.035 106.910442) (width 0.25) (layer B.Cu) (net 8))
 (segment (start 149.987 119.413) (end 149.987 109.958442) (width 0.25) (layer B.Cu) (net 8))
 (segment (start 153.035 103.379998) (end 154.934497 101.480501) (width 0.25) (layer B.Cu) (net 8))
 (segment (start 153.035 106.910442) (end 153.035 103.379998) (width 0.25) (layer B.Cu) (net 8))
 (segment (start 150.749 80.01) (end 157.48 80.01) (width 0.25) (layer B.Cu) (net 6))
 (segment (start 145.034 85.725) (end 150.749 80.01) (width 0.25) (layer B.Cu) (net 6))
 (segment (start 145.034 97.686998) (end 145.034 85.725) (width 0.25) (layer B.Cu) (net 6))
 (segment (start 152.781 122.916) (end 151.364 124.333) (width 0.25) (layer B.Cu) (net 6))
 (segment (start 152.781 121.666) (end 152.781 122.916) (width 0.25) (layer B.Cu) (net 6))
 (segment (start 151.364 124.333) (end 148.486998 124.333) (width 0.25) (layer B.Cu) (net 6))
 (segment (start 148.486998 124.333) (end 141.732 117.578002) (width 0.25) (layer B.Cu) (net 6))
 (segment (start 141.732 117.578002) (end 141.732 100.988998) (width 0.25) (layer B.Cu) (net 6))
 (segment (start 141.732 100.988998) (end 145.034 97.686998) (width 0.25) (layer B.Cu) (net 6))
 (segment (start 143.039999 73.189999) (end 142.24 72.39) (width 0.25) (layer B.Cu) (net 19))
 (segment (start 143.365001 73.515001) (end 143.039999 73.189999) (width 0.25) (layer B.Cu) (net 19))
 (segment (start 143.365001 75.470001) (end 143.365001 73.515001) (width 0.25) (layer B.Cu) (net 19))
 (segment (start 142.515002 76.32) (end 143.365001 75.470001) (width 0.25) (layer B.Cu) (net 19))
 (segment (start 133.31 76.32) (end 142.515002 76.32) (width 0.25) (layer B.Cu) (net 19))
 (segment (start 127.9417 76.8458) (end 130.9497 73.8378) (width 0.25) (layer B.Cu) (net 20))
 (segment (start 139.318802 73.8378) (end 140.6525 72.504102) (width 0.25) (layer B.Cu) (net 20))
 (segment (start 130.9497 73.8378) (end 139.318802 73.8378) (width 0.25) (layer B.Cu) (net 20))
 (segment (start 141.19 69.85) (end 142.24 69.85) (width 0.25) (layer B.Cu) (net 20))
 (segment (start 140.6525 70.3875) (end 141.19 69.85) (width 0.25) (layer B.Cu) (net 20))
 (segment (start 140.6525 72.504102) (end 140.6525 70.3875) (width 0.25) (layer B.Cu) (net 20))
 (segment (start 147.36 109.725787) (end 147.36 111.14) (width 0.25) (layer F.Cu) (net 2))
 (segment (start 147.36 101.244998) (end 147.36 109.725787) (width 0.25) (layer F.Cu) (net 2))
 (segment (start 142.24 96.124998) (end 147.36 101.244998) (width 0.25) (layer F.Cu) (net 2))
 (segment (start 142.24 95.25) (end 142.24 96.124998) (width 0.25) (layer F.Cu) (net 2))
 (segment (start 172.014001 119.632999) (end 173.014 118.633) (width 0.25) (layer F.Cu) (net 2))
 (segment (start 168.281999 123.365001) (end 172.014001 119.632999) (width 0.25) (layer F.Cu) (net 2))
 (segment (start 146.723999 123.365001) (end 168.281999 123.365001) (width 0.25) (layer F.Cu) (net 2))
 (segment (start 146.034999 122.676001) (end 146.723999 123.365001) (width 0.25) (layer F.Cu) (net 2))
 (segment (start 146.034999 112.465001) (end 146.034999 122.676001) (width 0.25) (layer F.Cu) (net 2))
 (segment (start 147.36 111.14) (end 146.034999 112.465001) (width 0.25) (layer F.Cu) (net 2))
 (segment (start 172.014001 117.633001) (end 173.014 118.633) (width 0.25) (layer F.Cu) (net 2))
 (segment (start 168.588999 114.207999) (end 172.014001 117.633001) (width 0.25) (layer F.Cu) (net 2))
 (segment (start 168.588999 95.538999) (end 168.588999 114.207999) (width 0.25) (layer F.Cu) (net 2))
 (segment (start 163.87 90.82) (end 168.588999 95.538999) (width 0.25) (layer F.Cu) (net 2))
 (segment (start 156.680001 86.830001) (end 157.48 87.63) (width 0.25) (layer F.Cu) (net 17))
 (segment (start 156.354999 86.504999) (end 156.680001 86.830001) (width 0.25) (layer F.Cu) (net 17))
 (segment (start 156.354999 76.929999) (end 156.354999 86.504999) (width 0.25) (layer F.Cu) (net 17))
 (segment (start 156.964998 76.32) (end 156.354999 76.929999) (width 0.25) (layer F.Cu) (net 17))
 (segment (start 163.87 76.32) (end 156.964998 76.32) (width 0.25) (layer F.Cu) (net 17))
 (segment (start 169.037 76.561) (end 163.175 82.423) (width 0.25) (layer F.Cu) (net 16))
 (segment (start 169.037 75.311) (end 169.037 76.561) (width 0.25) (layer F.Cu) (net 16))
 (segment (start 160.147 82.423) (end 157.48 85.09) (width 0.25) (layer F.Cu) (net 16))
 (segment (start 163.175 82.423) (end 160.147 82.423) (width 0.25) (layer F.Cu) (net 16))
 (segment (start 156.34863 97.79) (end 154.95163 99.187) (width 0.25) (layer B.Cu) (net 11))
 (segment (start 157.48 97.79) (end 156.34863 97.79) (width 0.25) (layer B.Cu) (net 11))
 (segment (start 149.907 99.187) (end 147.36 96.64) (width 0.25) (layer B.Cu) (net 11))
 (segment (start 154.95163 99.187) (end 149.907 99.187) (width 0.25) (layer B.Cu) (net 11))
 (segment (start 156.09 96.64) (end 157.48 95.25) (width 0.25) (layer B.Cu) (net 10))
 (segment (start 152.36 96.64) (end 156.09 96.64) (width 0.25) (layer B.Cu) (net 10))
 (segment (start 136.203401 99.256009) (end 140.030511 95.428899) (width 0.25) (layer F.Cu) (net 13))
 (segment (start 130.71399 99.25601) (end 136.203401 99.256009) (width 0.25) (layer F.Cu) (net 13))
 (segment (start 126.96 104.26) (end 126.96 103.01) (width 0.25) (layer F.Cu) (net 13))
 (segment (start 126.96 103.01) (end 130.71399 99.25601) (width 0.25) (layer F.Cu) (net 13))
 (segment (start 140.030511 84.759489) (end 142.24 82.55) (width 0.25) (layer F.Cu) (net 13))
 (segment (start 140.030511 95.428899) (end 140.030511 84.759489) (width 0.25) (layer F.Cu) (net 13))
 (segment (start 121.96 104.26) (end 127.414 98.806) (width 0.25) (layer F.Cu) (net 14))
 (segment (start 127.414 98.806) (end 136.017 98.806) (width 0.25) (layer F.Cu) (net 14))
 (segment (start 141.440001 80.809999) (end 142.24 80.01) (width 0.25) (layer F.Cu) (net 14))
 (segment (start 139.580501 82.669499) (end 141.440001 80.809999) (width 0.25) (layer F.Cu) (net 14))
 (segment (start 139.580501 95.242499) (end 139.580501 82.669499) (width 0.25) (layer F.Cu) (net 14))
 (segment (start 136.017 98.806) (end 139.580501 95.242499) (width 0.25) (layer F.Cu) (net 14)))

